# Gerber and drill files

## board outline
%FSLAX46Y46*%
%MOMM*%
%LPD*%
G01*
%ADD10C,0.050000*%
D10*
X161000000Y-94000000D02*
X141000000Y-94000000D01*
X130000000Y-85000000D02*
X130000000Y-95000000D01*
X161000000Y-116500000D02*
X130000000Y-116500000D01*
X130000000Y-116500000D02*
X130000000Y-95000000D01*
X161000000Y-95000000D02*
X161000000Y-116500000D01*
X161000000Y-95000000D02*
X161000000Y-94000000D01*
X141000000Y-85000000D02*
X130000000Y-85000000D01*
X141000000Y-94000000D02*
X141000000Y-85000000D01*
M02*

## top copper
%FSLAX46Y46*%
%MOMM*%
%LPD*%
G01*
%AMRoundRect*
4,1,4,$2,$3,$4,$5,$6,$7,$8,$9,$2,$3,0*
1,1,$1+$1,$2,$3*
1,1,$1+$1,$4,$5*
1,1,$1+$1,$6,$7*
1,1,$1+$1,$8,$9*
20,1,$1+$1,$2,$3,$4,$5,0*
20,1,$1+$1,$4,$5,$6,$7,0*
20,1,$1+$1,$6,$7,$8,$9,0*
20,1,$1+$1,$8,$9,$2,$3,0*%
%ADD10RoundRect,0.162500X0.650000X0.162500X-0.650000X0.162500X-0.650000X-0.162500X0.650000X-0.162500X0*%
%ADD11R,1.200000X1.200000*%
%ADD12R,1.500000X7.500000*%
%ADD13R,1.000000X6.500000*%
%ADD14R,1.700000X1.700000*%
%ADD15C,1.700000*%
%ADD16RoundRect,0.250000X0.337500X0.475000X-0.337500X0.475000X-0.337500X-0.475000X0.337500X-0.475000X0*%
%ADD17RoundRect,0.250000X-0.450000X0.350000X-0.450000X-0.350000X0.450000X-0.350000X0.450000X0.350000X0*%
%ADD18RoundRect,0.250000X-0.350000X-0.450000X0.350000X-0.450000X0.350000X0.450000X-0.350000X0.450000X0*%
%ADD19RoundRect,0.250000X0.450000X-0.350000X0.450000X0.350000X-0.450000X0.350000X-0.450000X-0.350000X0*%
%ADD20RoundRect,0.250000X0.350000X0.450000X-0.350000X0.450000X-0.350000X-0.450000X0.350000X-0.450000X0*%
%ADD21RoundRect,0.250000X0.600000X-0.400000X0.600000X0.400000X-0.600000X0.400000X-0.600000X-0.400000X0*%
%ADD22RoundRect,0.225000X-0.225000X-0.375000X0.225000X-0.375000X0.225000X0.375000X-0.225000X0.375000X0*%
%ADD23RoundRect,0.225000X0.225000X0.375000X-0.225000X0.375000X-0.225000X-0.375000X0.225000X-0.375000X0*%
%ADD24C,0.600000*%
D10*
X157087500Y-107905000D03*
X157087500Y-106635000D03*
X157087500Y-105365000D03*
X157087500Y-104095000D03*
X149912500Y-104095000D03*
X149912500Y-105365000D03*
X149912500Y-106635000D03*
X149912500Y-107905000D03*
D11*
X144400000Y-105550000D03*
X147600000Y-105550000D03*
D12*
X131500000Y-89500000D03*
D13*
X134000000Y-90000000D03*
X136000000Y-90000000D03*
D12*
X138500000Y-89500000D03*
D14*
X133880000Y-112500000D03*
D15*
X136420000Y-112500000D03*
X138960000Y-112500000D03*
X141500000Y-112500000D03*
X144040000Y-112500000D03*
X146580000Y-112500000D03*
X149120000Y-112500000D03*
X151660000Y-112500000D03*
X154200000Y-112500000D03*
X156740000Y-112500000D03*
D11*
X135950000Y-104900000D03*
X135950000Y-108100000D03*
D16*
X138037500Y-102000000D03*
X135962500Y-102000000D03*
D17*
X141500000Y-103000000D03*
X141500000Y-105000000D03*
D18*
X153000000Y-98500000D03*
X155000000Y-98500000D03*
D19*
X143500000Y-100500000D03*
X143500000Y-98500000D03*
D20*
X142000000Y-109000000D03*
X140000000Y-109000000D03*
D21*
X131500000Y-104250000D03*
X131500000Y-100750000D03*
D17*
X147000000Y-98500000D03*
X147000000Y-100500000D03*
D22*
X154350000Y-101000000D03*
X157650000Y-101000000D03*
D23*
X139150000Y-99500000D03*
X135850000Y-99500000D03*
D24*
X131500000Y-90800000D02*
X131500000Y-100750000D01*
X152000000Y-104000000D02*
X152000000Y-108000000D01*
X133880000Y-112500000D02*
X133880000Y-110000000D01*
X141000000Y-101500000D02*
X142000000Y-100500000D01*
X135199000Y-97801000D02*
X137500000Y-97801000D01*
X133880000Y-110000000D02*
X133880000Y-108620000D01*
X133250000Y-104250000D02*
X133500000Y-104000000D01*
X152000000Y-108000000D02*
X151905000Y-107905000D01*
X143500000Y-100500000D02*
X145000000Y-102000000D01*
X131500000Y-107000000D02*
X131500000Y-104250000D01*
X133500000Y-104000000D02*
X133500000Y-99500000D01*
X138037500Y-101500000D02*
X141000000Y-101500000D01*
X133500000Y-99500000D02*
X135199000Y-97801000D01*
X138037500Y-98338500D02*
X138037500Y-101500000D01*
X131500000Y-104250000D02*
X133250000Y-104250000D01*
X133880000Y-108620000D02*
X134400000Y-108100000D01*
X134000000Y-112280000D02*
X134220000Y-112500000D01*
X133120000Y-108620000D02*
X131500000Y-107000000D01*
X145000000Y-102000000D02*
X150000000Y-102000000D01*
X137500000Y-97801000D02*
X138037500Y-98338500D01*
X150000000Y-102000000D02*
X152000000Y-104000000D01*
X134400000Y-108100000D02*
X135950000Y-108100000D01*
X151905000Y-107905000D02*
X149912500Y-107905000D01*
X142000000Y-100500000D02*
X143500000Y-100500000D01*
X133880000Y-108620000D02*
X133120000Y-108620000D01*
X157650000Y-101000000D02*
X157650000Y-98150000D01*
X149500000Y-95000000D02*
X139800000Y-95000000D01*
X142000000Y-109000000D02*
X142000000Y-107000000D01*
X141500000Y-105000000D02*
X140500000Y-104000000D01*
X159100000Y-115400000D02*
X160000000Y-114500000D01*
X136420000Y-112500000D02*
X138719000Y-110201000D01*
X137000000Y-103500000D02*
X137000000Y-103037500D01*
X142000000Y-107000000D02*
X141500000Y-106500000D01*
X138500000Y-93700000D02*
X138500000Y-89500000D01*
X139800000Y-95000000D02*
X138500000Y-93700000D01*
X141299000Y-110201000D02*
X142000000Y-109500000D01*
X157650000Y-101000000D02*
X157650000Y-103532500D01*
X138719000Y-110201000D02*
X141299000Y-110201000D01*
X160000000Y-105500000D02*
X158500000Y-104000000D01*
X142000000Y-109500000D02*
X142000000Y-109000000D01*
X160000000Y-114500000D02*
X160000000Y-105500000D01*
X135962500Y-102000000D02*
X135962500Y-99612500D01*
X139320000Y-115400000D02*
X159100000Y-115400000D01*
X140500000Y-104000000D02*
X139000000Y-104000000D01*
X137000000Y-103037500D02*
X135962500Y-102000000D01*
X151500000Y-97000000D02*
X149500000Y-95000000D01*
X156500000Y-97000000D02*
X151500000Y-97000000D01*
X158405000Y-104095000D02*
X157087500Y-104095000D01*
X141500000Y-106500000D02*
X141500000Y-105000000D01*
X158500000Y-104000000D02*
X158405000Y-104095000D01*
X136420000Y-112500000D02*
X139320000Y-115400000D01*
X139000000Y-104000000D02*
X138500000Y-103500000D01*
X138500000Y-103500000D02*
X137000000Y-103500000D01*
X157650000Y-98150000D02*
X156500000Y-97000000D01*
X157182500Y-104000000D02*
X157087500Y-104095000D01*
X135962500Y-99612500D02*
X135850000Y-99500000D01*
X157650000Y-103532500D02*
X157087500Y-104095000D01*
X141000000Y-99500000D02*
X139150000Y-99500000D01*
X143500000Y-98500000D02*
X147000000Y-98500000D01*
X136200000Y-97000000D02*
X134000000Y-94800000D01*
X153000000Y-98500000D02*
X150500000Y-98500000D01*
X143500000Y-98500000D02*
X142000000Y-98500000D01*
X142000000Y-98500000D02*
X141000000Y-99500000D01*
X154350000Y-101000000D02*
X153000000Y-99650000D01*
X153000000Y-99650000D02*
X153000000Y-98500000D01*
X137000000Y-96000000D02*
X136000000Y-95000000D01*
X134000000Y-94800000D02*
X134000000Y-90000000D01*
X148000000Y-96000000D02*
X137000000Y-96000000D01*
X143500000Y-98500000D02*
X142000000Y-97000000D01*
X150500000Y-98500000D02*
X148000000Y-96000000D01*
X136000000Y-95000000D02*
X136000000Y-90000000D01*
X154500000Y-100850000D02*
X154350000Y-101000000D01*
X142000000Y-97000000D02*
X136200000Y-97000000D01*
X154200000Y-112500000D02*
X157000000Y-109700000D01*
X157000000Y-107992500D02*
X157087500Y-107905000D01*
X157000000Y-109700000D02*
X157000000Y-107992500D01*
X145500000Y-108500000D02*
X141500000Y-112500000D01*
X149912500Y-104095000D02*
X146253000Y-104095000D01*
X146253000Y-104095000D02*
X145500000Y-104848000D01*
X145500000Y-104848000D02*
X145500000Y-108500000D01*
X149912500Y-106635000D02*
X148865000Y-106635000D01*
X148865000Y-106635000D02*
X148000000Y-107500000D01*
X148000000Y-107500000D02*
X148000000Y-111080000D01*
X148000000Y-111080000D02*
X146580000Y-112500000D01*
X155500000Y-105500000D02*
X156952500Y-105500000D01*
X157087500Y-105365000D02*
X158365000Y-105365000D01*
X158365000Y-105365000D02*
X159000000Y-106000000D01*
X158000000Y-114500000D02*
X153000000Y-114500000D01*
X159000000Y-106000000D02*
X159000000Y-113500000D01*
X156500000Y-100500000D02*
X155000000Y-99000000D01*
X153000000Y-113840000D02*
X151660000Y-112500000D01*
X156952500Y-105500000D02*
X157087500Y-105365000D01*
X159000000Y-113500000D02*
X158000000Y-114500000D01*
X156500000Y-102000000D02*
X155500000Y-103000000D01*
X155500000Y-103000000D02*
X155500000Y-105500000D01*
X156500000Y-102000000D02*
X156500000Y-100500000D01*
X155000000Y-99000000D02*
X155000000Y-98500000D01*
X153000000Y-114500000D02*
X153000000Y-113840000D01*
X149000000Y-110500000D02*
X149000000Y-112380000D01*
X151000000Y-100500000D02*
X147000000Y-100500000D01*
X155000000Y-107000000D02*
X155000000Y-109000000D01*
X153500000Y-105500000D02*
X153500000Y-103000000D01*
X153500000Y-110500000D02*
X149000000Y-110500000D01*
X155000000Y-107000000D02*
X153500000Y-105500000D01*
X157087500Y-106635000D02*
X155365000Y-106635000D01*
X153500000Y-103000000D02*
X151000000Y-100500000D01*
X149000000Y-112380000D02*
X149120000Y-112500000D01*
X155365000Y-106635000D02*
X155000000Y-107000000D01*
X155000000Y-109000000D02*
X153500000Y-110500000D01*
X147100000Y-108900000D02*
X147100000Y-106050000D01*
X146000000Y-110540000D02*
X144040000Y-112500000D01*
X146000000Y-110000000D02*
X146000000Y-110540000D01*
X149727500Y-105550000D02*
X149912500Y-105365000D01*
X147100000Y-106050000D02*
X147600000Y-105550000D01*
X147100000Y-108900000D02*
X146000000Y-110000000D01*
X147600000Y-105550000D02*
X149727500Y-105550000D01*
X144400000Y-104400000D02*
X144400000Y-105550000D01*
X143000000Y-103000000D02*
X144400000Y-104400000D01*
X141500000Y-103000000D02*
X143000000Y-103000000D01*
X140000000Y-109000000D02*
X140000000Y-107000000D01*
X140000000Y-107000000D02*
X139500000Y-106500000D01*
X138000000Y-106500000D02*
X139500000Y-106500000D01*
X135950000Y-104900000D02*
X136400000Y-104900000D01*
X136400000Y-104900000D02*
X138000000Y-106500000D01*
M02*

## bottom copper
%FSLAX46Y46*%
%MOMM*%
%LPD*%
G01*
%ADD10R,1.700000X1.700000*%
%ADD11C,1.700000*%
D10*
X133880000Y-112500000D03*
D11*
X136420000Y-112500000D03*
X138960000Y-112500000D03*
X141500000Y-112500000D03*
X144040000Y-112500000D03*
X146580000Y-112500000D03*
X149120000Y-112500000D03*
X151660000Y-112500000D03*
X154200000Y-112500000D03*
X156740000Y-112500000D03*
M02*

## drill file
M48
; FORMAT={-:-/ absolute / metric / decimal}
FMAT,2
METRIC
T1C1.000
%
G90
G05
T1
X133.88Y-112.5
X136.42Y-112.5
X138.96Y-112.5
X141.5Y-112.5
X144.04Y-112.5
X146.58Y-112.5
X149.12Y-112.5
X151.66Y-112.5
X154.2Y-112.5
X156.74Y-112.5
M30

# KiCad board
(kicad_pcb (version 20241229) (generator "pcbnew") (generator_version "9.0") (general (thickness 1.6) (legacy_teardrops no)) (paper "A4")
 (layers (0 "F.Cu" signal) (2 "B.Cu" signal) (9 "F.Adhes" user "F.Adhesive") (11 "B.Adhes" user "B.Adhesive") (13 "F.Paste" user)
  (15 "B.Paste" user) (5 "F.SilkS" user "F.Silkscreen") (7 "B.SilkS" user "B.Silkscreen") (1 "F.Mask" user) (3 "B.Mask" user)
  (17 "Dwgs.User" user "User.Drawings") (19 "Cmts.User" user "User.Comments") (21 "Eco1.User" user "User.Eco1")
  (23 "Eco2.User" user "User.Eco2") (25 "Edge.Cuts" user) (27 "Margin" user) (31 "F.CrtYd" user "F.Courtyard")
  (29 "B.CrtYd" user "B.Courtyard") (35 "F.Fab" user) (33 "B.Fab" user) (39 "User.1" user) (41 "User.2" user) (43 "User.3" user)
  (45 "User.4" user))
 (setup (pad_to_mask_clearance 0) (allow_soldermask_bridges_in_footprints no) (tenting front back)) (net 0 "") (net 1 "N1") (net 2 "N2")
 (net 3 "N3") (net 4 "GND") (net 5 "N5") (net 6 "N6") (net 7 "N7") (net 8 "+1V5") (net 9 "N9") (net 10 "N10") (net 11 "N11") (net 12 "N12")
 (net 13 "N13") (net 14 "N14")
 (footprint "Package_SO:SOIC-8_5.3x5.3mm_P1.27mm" (layer "F.Cu") (at 153.5 106 180)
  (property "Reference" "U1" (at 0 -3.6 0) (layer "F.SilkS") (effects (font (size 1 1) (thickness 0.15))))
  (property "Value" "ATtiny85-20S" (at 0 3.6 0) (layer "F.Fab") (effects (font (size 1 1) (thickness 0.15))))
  (pad "1" smd roundrect (at -3.5875 -1.905 180) (size 1.625 0.65) (layers "F.Cu" "F.Mask" "F.Paste") (roundrect_rratio 0.25) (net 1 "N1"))
  (pad "2" smd roundrect (at -3.5875 -0.635 180) (size 1.625 0.65) (layers "F.Cu" "F.Mask" "F.Paste") (roundrect_rratio 0.25) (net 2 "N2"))
  (pad "3" smd roundrect (at -3.5875 0.635 180) (size 1.625 0.65) (layers "F.Cu" "F.Mask" "F.Paste") (roundrect_rratio 0.25) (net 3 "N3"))
  (pad "4" smd roundrect (at -3.5875 1.905 180) (size 1.625 0.65) (layers "F.Cu" "F.Mask" "F.Paste") (roundrect_rratio 0.25) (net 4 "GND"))
  (pad "5" smd roundrect (at 3.5875 1.905 180) (size 1.625 0.65) (layers "F.Cu" "F.Mask" "F.Paste") (roundrect_rratio 0.25) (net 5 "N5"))
  (pad "6" smd roundrect (at 3.5875 0.635 180) (size 1.625 0.65) (layers "F.Cu" "F.Mask" "F.Paste") (roundrect_rratio 0.25) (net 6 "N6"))
  (pad "7" smd roundrect (at 3.5875 -0.635 180) (size 1.625 0.65) (layers "F.Cu" "F.Mask" "F.Paste") (roundrect_rratio 0.25) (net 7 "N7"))
  (pad "8" smd roundrect (at 3.5875 -1.905 180) (size 1.625 0.65) (layers "F.Cu" "F.Mask" "F.Paste") (roundrect_rratio 0.25) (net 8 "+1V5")))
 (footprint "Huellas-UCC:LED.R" (layer "F.Cu") (at 146.5 105.1)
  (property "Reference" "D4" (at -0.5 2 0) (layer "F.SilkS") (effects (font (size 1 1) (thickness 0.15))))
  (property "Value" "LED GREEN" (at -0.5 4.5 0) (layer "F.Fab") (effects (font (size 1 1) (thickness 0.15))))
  (pad "1" smd rect (at -2.1 0.45) (size 1.2 1.2) (layers "F.Cu" "F.Mask" "F.Paste") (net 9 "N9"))
  (pad "2" smd rect (at 1.1 0.45) (size 1.2 1.2) (layers "F.Cu" "F.Mask" "F.Paste") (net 6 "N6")))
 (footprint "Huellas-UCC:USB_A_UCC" (layer "F.Cu") (at 135 89.7 -90)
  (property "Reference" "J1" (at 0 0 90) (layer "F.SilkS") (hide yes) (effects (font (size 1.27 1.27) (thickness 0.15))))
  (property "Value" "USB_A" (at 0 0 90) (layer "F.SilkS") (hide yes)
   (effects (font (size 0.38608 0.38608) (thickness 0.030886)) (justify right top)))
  (pad "1" smd rect (at -0.2 3.5 270) (size 7.5 1.5) (layers "F.Cu" "F.Mask" "F.Paste") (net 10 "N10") (solder_mask_margin 0.1016))
  (pad "2" smd rect (at 0.3 1 270) (size 6.5 1) (layers "F.Cu" "F.Mask" "F.Paste") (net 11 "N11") (solder_mask_margin 0.1016))
  (pad "3" smd rect (at 0.3 -1 270) (size 6.5 1) (layers "F.Cu" "F.Mask" "F.Paste") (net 11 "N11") (solder_mask_margin 0.1016))
  (pad "4" smd rect (at -0.2 -3.5 270) (size 7.5 1.5) (layers "F.Cu" "F.Mask" "F.Paste") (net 4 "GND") (solder_mask_margin 0.1016)))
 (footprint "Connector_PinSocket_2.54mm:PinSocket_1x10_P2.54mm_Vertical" (layer "F.Cu") (at 133.88 112.5 90)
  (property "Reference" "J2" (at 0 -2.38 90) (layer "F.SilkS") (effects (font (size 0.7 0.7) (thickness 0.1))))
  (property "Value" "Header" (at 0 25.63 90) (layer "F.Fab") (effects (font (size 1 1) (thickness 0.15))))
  (pad "1" thru_hole rect (at 0 0 90) (size 1.7 1.7) (drill 1) (layers "*.Cu" "*.Mask") (remove_unused_layers no) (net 8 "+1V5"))
  (pad "2" thru_hole circle (at 0 2.54 90) (size 1.7 1.7) (drill 1) (layers "*.Cu" "*.Mask") (remove_unused_layers no) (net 4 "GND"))
  (pad "3" thru_hole circle (at 0 5.08 90) (size 1.7 1.7) (drill 1) (layers "*.Cu" "*.Mask") (remove_unused_layers no) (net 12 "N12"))
  (pad "4" thru_hole circle (at 0 7.62 90) (size 1.7 1.7) (drill 1) (layers "*.Cu" "*.Mask") (remove_unused_layers no) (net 5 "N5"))
  (pad "5" thru_hole circle (at 0 10.16 90) (size 1.7 1.7) (drill 1) (layers "*.Cu" "*.Mask") (remove_unused_layers no) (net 6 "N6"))
  (pad "6" thru_hole circle (at 0 12.7 90) (size 1.7 1.7) (drill 1) (layers "*.Cu" "*.Mask") (remove_unused_layers no) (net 7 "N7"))
  (pad "7" thru_hole circle (at 0 15.24 90) (size 1.7 1.7) (drill 1) (layers "*.Cu" "*.Mask") (remove_unused_layers no) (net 2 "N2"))
  (pad "8" thru_hole circle (at 0 17.78 90) (size 1.7 1.7) (drill 1) (layers "*.Cu" "*.Mask") (remove_unused_layers no) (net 3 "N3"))
  (pad "9" thru_hole circle (at 0 20.32 90) (size 1.7 1.7) (drill 1) (layers "*.Cu" "*.Mask") (remove_unused_layers no) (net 1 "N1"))
  (pad "10" thru_hole circle (at 0 22.86 90) (size 1.7 1.7) (drill 1) (layers "*.Cu" "*.Mask") (remove_unused_layers no) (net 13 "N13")))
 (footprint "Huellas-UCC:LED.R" (layer "F.Cu") (at 136.4 107 -90)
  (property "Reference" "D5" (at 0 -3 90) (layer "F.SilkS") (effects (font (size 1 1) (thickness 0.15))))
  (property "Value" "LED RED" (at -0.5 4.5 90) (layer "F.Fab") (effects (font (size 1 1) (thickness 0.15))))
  (pad "1" smd rect (at -2.1 0.45 270) (size 1.2 1.2) (layers "F.Cu" "F.Mask" "F.Paste") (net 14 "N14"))
  (pad "2" smd rect (at 1.1 0.45 270) (size 1.2 1.2) (layers "F.Cu" "F.Mask" "F.Paste") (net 8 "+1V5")))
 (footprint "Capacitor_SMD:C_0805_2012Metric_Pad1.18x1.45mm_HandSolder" (layer "F.Cu") (at 137 102 180)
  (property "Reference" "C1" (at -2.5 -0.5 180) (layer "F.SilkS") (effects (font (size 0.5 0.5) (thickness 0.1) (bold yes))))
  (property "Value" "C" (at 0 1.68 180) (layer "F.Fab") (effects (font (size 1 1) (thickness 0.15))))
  (pad "1" smd roundrect (at -1.0375 0 180) (size 1.175 1.45) (layers "F.Cu" "F.Mask" "F.Paste") (roundrect_rratio 0.212766) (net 8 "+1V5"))
  (pad "2" smd roundrect (at 1.0375 0 180) (size 1.175 1.45) (layers "F.Cu" "F.Mask" "F.Paste") (roundrect_rratio 0.212766) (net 4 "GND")))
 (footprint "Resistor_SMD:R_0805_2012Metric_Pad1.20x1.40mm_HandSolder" (layer "F.Cu") (at 141.5 104 -90)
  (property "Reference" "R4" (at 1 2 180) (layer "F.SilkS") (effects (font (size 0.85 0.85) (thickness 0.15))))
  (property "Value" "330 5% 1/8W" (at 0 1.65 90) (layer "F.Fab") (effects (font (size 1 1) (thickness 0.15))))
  (pad "1" smd roundrect (at -1 0 270) (size 1.2 1.4) (layers "F.Cu" "F.Mask" "F.Paste") (roundrect_rratio 0.208333) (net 9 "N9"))
  (pad "2" smd roundrect (at 1 0 270) (size 1.2 1.4) (layers "F.Cu" "F.Mask" "F.Paste") (roundrect_rratio 0.208333) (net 4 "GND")))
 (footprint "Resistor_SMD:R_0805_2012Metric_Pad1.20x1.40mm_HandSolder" (layer "F.Cu") (at 154 98.5)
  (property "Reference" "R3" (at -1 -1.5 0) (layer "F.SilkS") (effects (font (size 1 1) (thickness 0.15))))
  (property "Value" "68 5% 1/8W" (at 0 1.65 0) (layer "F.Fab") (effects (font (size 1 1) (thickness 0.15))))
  (pad "1" smd roundrect (at -1 0) (size 1.2 1.4) (layers "F.Cu" "F.Mask" "F.Paste") (roundrect_rratio 0.208333) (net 11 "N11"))
  (pad "2" smd roundrect (at 1 0) (size 1.2 1.4) (layers "F.Cu" "F.Mask" "F.Paste") (roundrect_rratio 0.208333) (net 3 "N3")))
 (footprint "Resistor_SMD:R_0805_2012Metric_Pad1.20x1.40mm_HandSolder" (layer "F.Cu") (at 143.5 99.5 90)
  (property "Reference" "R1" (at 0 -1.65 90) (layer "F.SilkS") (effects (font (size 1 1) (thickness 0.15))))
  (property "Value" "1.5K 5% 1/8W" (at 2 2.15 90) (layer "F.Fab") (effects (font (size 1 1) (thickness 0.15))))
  (pad "1" smd roundrect (at -1 0 90) (size 1.2 1.4) (layers "F.Cu" "F.Mask" "F.Paste") (roundrect_rratio 0.208333) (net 8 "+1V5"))
  (pad "2" smd roundrect (at 1 0 90) (size 1.2 1.4) (layers "F.Cu" "F.Mask" "F.Paste") (roundrect_rratio 0.208333) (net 11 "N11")))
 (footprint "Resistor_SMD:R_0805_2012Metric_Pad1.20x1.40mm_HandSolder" (layer "F.Cu") (at 141 109 180)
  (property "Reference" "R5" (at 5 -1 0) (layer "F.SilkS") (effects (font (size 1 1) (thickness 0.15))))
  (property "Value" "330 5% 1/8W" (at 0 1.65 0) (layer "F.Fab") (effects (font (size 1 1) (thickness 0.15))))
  (pad "1" smd roundrect (at -1 0 180) (size 1.2 1.4) (layers "F.Cu" "F.Mask" "F.Paste") (roundrect_rratio 0.208333) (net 4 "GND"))
  (pad "2" smd roundrect (at 1 0 180) (size 1.2 1.4) (layers "F.Cu" "F.Mask" "F.Paste") (roundrect_rratio 0.208333) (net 14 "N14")))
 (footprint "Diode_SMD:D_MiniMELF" (layer "F.Cu") (at 131.5 102.5 90)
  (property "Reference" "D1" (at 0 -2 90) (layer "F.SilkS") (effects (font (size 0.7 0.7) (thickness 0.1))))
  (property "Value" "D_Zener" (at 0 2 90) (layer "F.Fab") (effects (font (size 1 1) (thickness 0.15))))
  (pad "1" smd roundrect (at -1.75 0 90) (size 1.3 1.7) (layers "F.Cu" "F.Mask" "F.Paste") (roundrect_rratio 0.1923076923) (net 8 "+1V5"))
  (pad "2" smd roundrect (at 1.75 0 90) (size 1.3 1.7) (layers "F.Cu" "F.Mask" "F.Paste") (roundrect_rratio 0.1923076923) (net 10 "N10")))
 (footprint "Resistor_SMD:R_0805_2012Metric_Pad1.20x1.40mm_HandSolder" (layer "F.Cu") (at 147 99.5 -90)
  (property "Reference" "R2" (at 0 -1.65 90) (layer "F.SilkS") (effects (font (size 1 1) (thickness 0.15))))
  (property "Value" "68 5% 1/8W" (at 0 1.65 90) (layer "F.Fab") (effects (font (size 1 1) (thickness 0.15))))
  (pad "1" smd roundrect (at -1 0 270) (size 1.2 1.4) (layers "F.Cu" "F.Mask" "F.Paste") (roundrect_rratio 0.208333) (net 11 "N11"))
  (pad "2" smd roundrect (at 1 0 270) (size 1.2 1.4) (layers "F.Cu" "F.Mask" "F.Paste") (roundrect_rratio 0.208333) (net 2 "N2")))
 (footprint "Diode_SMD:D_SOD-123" (layer "F.Cu") (at 156 101)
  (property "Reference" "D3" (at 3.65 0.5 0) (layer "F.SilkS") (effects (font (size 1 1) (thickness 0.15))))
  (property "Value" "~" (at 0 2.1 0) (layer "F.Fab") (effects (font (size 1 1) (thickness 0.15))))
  (pad "1" smd roundrect (at -1.65 0) (size 0.9 1.2) (layers "F.Cu" "F.Mask" "F.Paste") (roundrect_rratio 0.25) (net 11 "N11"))
  (pad "2" smd roundrect (at 1.65 0) (size 0.9 1.2) (layers "F.Cu" "F.Mask" "F.Paste") (roundrect_rratio 0.25) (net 4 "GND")))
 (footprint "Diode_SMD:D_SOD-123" (layer "F.Cu") (at 137.5 99.5 180)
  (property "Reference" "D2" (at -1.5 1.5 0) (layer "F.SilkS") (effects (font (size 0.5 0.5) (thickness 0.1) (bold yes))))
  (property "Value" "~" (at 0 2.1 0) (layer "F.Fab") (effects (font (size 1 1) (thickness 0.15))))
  (pad "1" smd roundrect (at -1.65 0 180) (size 0.9 1.2) (layers "F.Cu" "F.Mask" "F.Paste") (roundrect_rratio 0.25) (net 11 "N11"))
  (pad "2" smd roundrect (at 1.65 0 180) (size 0.9 1.2) (layers "F.Cu" "F.Mask" "F.Paste") (roundrect_rratio 0.25) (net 4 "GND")))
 (gr_line (start 161 94) (end 141 94) (stroke (width 0.05) (type default)) (layer "Edge.Cuts"))
 (gr_line (start 130 85) (end 130 95) (stroke (width 0.05) (type default)) (layer "Edge.Cuts"))
 (gr_line (start 161 116.5) (end 130 116.5) (stroke (width 0.05) (type default)) (layer "Edge.Cuts"))
 (gr_line (start 130 116.5) (end 130 95) (stroke (width 0.05) (type default)) (layer "Edge.Cuts"))
 (gr_line (start 161 95) (end 161 116.5) (stroke (width 0.05) (type default)) (layer "Edge.Cuts"))
 (gr_line (start 161 95) (end 161 94) (stroke (width 0.05) (type default)) (layer "Edge.Cuts"))
 (gr_line (start 141 85) (end 130 85) (stroke (width 0.05) (type default)) (layer "Edge.Cuts"))
 (gr_line (start 141 94) (end 141 85) (stroke (width 0.05) (type default)) (layer "Edge.Cuts"))
 (segment (start 131.5 90.8) (end 131.5 100.75) (width 0.6) (layer "F.Cu") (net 10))
 (segment (start 152 104) (end 152 108) (width 0.6) (layer "F.Cu") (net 8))
 (segment (start 133.88 112.5) (end 133.88 110) (width 0.6) (layer "F.Cu") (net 8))
 (segment (start 141 101.5) (end 142 100.5) (width 0.6) (layer "F.Cu") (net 8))
 (segment (start 135.199 97.801) (end 137.5 97.801) (width 0.6) (layer "F.Cu") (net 8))
 (segment (start 133.88 110) (end 133.88 108.62) (width 0.6) (layer "F.Cu") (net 8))
 (segment (start 133.25 104.25) (end 133.5 104) (width 0.6) (layer "F.Cu") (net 8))
 (segment (start 152 108) (end 151.905 107.905) (width 0.6) (layer "F.Cu") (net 8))
 (segment (start 143.5 100.5) (end 145 102) (width 0.6) (layer "F.Cu") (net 8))
 (segment (start 131.5 107) (end 131.5 104.25) (width 0.6) (layer "F.Cu") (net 8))
 (segment (start 133.5 104) (end 133.5 99.5) (width 0.6) (layer "F.Cu") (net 8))
 (segment (start 138.0375 101.5) (end 141 101.5) (width 0.6) (layer "F.Cu") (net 8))
 (segment (start 133.5 99.5) (end 135.199 97.801) (width 0.6) (layer "F.Cu") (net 8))
 (segment (start 138.0375 98.3385) (end 138.0375 101.5) (width 0.6) (layer "F.Cu") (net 8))
 (segment (start 131.5 104.25) (end 133.25 104.25) (width 0.6) (layer "F.Cu") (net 8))
 (segment (start 133.88 108.62) (end 134.4 108.1) (width 0.6) (layer "F.Cu") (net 8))
 (segment (start 134 112.28) (end 134.22 112.5) (width 0.6) (layer "F.Cu") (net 8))
 (segment (start 133.12 108.62) (end 131.5 107) (width 0.6) (layer "F.Cu") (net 8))
 (segment (start 145 102) (end 150 102) (width 0.6) (layer "F.Cu") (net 8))
 (segment (start 137.5 97.801) (end 138.0375 98.3385) (width 0.6) (layer "F.Cu") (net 8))
 (segment (start 150 102) (end 152 104) (width 0.6) (layer "F.Cu") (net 8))
 (segment (start 134.4 108.1) (end 135.95 108.1) (width 0.6) (layer "F.Cu") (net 8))
 (segment (start 151.905 107.905) (end 149.9125 107.905) (width 0.6) (layer "F.Cu") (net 8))
 (segment (start 142 100.5) (end 143.5 100.5) (width 0.6) (layer "F.Cu") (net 8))
 (segment (start 133.88 108.62) (end 133.12 108.62) (width 0.6) (layer "F.Cu") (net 8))
 (segment (start 157.65 101) (end 157.65 98.15) (width 0.6) (layer "F.Cu") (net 4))
 (segment (start 149.5 95) (end 139.8 95) (width 0.6) (layer "F.Cu") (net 4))
 (segment (start 142 109) (end 142 107) (width 0.6) (layer "F.Cu") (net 4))
 (segment (start 141.5 105) (end 140.5 104) (width 0.6) (layer "F.Cu") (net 4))
 (segment (start 159.1 115.4) (end 160 114.5) (width 0.6) (layer "F.Cu") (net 4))
 (segment (start 136.42 112.5) (end 138.719 110.201) (width 0.6) (layer "F.Cu") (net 4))
 (segment (start 137 103.5) (end 137 103.0375) (width 0.6) (layer "F.Cu") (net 4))
 (segment (start 142 107) (end 141.5 106.5) (width 0.6) (layer "F.Cu") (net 4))
 (segment (start 138.5 93.7) (end 138.5 89.5) (width 0.6) (layer "F.Cu") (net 4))
 (segment (start 139.8 95) (end 138.5 93.7) (width 0.6) (layer "F.Cu") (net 4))
 (segment (start 141.299 110.201) (end 142 109.5) (width 0.6) (layer "F.Cu") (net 4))
 (segment (start 157.65 101) (end 157.65 103.5325) (width 0.6) (layer "F.Cu") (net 4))
 (segment (start 138.719 110.201) (end 141.299 110.201) (width 0.6) (layer "F.Cu") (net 4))
 (segment (start 160 105.5) (end 158.5 104) (width 0.6) (layer "F.Cu") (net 4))
 (segment (start 142 109.5) (end 142 109) (width 0.6) (layer "F.Cu") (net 4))
 (segment (start 160 114.5) (end 160 105.5) (width 0.6) (layer "F.Cu") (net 4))
 (segment (start 135.9625 102) (end 135.9625 99.6125) (width 0.6) (layer "F.Cu") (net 4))
 (segment (start 139.32 115.4) (end 159.1 115.4) (width 0.6) (layer "F.Cu") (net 4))
 (segment (start 140.5 104) (end 139 104) (width 0.6) (layer "F.Cu") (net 4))
 (segment (start 137 103.0375) (end 135.9625 102) (width 0.6) (layer "F.Cu") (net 4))
 (segment (start 151.5 97) (end 149.5 95) (width 0.6) (layer "F.Cu") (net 4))
 (segment (start 156.5 97) (end 151.5 97) (width 0.6) (layer "F.Cu") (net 4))
 (segment (start 158.405 104.095) (end 157.0875 104.095) (width 0.6) (layer "F.Cu") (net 4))
 (segment (start 141.5 106.5) (end 141.5 105) (width 0.6) (layer "F.Cu") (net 4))
 (segment (start 158.5 104) (end 158.405 104.095) (width 0.6) (layer "F.Cu") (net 4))
 (segment (start 136.42 112.5) (end 139.32 115.4) (width 0.6) (layer "F.Cu") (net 4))
 (segment (start 139 104) (end 138.5 103.5) (width 0.6) (layer "F.Cu") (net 4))
 (segment (start 138.5 103.5) (end 137 103.5) (width 0.6) (layer "F.Cu") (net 4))
 (segment (start 157.65 98.15) (end 156.5 97) (width 0.6) (layer "F.Cu") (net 4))
 (segment (start 157.1825 104) (end 157.0875 104.095) (width 0.6) (layer "F.Cu") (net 4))
 (segment (start 135.9625 99.6125) (end 135.85 99.5) (width 0.6) (layer "F.Cu") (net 4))
 (segment (start 157.65 103.5325) (end 157.0875 104.095) (width 0.6) (layer "F.Cu") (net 4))
 (segment (start 141 99.5) (end 139.15 99.5) (width 0.6) (layer "F.Cu") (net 11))
 (segment (start 143.5 98.5) (end 147 98.5) (width 0.6) (layer "F.Cu") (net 11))
 (segment (start 136.2 97) (end 134 94.8) (width 0.6) (layer "F.Cu") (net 11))
 (segment (start 153 98.5) (end 150.5 98.5) (width 0.6) (layer "F.Cu") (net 11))
 (segment (start 143.5 98.5) (end 142 98.5) (width 0.6) (layer "F.Cu") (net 11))
 (segment (start 142 98.5) (end 141 99.5) (width 0.6) (layer "F.Cu") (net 11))
 (segment (start 154.35 101) (end 153 99.65) (width 0.6) (layer "F.Cu") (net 11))
 (segment (start 153 99.65) (end 153 98.5) (width 0.6) (layer "F.Cu") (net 11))
 (segment (start 137 96) (end 136 95) (width 0.6) (layer "F.Cu") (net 11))
 (segment (start 134 94.8) (end 134 90) (width 0.6) (layer "F.Cu") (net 11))
 (segment (start 148 96) (end 137 96) (width 0.6) (layer "F.Cu") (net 11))
 (segment (start 143.5 98.5) (end 142 97) (width 0.6) (layer "F.Cu") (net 11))
 (segment (start 150.5 98.5) (end 148 96) (width 0.6) (layer "F.Cu") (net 11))
 (segment (start 136 95) (end 136 90) (width 0.6) (layer "F.Cu") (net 11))
 (segment (start 154.5 100.85) (end 154.35 101) (width 0.6) (layer "F.Cu") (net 11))
 (segment (start 142 97) (end 136.2 97) (width 0.6) (layer "F.Cu") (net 11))
 (segment (start 154.2 112.5) (end 157 109.7) (width 0.6) (layer "F.Cu") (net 1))
 (segment (start 157 107.9925) (end 157.0875 107.905) (width 0.6) (layer "F.Cu") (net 1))
 (segment (start 157 109.7) (end 157 107.9925) (width 0.6) (layer "F.Cu") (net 1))
 (segment (start 145.5 108.5) (end 141.5 112.5) (width 0.6) (layer "F.Cu") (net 5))
 (segment (start 149.9125 104.095) (end 146.253 104.095) (width 0.6) (layer "F.Cu") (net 5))
 (segment (start 146.253 104.095) (end 145.5 104.848) (width 0.6) (layer "F.Cu") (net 5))
 (segment (start 145.5 104.848) (end 145.5 108.5) (width 0.6) (layer "F.Cu") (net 5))
 (segment (start 149.9125 106.635) (end 148.865 106.635) (width 0.6) (layer "F.Cu") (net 7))
 (segment (start 148.865 106.635) (end 148 107.5) (width 0.6) (layer "F.Cu") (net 7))
 (segment (start 148 107.5) (end 148 111.08) (width 0.6) (layer "F.Cu") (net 7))
 (segment (start 148 111.08) (end 146.58 112.5) (width 0.6) (layer "F.Cu") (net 7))
 (segment (start 155.5 105.5) (end 156.9525 105.5) (width 0.6) (layer "F.Cu") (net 3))
 (segment (start 157.0875 105.365) (end 158.365 105.365) (width 0.6) (layer "F.Cu") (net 3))
 (segment (start 158.365 105.365) (end 159 106) (width 0.6) (layer "F.Cu") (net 3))
 (segment (start 158 114.5) (end 153 114.5) (width 0.6) (layer "F.Cu") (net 3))
 (segment (start 159 106) (end 159 113.5) (width 0.6) (layer "F.Cu") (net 3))
 (segment (start 156.5 100.5) (end 155 99) (width 0.6) (layer "F.Cu") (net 3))
 (segment (start 153 113.84) (end 151.66 112.5) (width 0.6) (layer "F.Cu") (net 3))
 (segment (start 156.9525 105.5) (end 157.0875 105.365) (width 0.6) (layer "F.Cu") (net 3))
 (segment (start 159 113.5) (end 158 114.5) (width 0.6) (layer "F.Cu") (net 3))
 (segment (start 156.5 102) (end 155.5 103) (width 0.6) (layer "F.Cu") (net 3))
 (segment (start 155.5 103) (end 155.5 105.5) (width 0.6) (layer "F.Cu") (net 3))
 (segment (start 156.5 102) (end 156.5 100.5) (width 0.6) (layer "F.Cu") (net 3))
 (segment (start 155 99) (end 155 98.5) (width 0.6) (layer "F.Cu") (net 3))
 (segment (start 153 114.5) (end 153 113.84) (width 0.6) (layer "F.Cu") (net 3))
 (segment (start 149 110.5) (end 149 112.38) (width 0.6) (layer "F.Cu") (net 2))
 (segment (start 151 100.5) (end 147 100.5) (width 0.6) (layer "F.Cu") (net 2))
 (segment (start 155 107) (end 155 109) (width 0.6) (layer "F.Cu") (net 2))
 (segment (start 153.5 105.5) (end 153.5 103) (width 0.6) (layer "F.Cu") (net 2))
 (segment (start 153.5 110.5) (end 149 110.5) (width 0.6) (layer "F.Cu") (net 2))
 (segment (start 155 107) (end 153.5 105.5) (width 0.6) (layer "F.Cu") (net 2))
 (segment (start 157.0875 106.635) (end 155.365 106.635) (width 0.6) (layer "F.Cu") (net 2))
 (segment (start 153.5 103) (end 151 100.5) (width 0.6) (layer "F.Cu") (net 2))
 (segment (start 149 112.38) (end 149.12 112.5) (width 0.6) (layer "F.Cu") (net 2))
 (segment (start 155.365 106.635) (end 155 107) (width 0.6) (layer "F.Cu") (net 2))
 (segment (start 155 109) (end 153.5 110.5) (width 0.6) (layer "F.Cu") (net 2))
 (segment (start 147.1 108.9) (end 147.1 106.05) (width 0.6) (layer "F.Cu") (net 6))
 (segment (start 146 110.54) (end 144.04 112.5) (width 0.6) (layer "F.Cu") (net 6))
 (segment (start 146 110) (end 146 110.54) (width 0.6) (layer "F.Cu") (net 6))
 (segment (start 149.7275 105.55) (end 149.9125 105.365) (width 0.6) (layer "F.Cu") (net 6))
 (segment (start 147.1 106.05) (end 147.6 105.55) (width 0.6) (layer "F.Cu") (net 6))
 (segment (start 147.1 108.9) (end 146 110) (width 0.6) (layer "F.Cu") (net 6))
 (segment (start 147.6 105.55) (end 149.7275 105.55) (width 0.6) (layer "F.Cu") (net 6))
 (segment (start 144.4 104.4) (end 144.4 105.55) (width 0.6) (layer "F.Cu") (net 9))
 (segment (start 143 103) (end 144.4 104.4) (width 0.6) (layer "F.Cu") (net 9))
 (segment (start 141.5 103) (end 143 103) (width 0.6) (layer "F.Cu") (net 9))
 (segment (start 140 109) (end 140 107) (width 0.6) (layer "F.Cu") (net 14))
 (segment (start 140 107) (end 139.5 106.5) (width 0.6) (layer "F.Cu") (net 14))
 (segment (start 138 106.5) (end 139.5 106.5) (width 0.6) (layer "F.Cu") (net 14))
 (segment (start 135.95 104.9) (end 136.4 104.9) (width 0.6) (layer "F.Cu") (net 14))
 (segment (start 136.4 104.9) (end 138 106.5) (width 0.6) (layer "F.Cu") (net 14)))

